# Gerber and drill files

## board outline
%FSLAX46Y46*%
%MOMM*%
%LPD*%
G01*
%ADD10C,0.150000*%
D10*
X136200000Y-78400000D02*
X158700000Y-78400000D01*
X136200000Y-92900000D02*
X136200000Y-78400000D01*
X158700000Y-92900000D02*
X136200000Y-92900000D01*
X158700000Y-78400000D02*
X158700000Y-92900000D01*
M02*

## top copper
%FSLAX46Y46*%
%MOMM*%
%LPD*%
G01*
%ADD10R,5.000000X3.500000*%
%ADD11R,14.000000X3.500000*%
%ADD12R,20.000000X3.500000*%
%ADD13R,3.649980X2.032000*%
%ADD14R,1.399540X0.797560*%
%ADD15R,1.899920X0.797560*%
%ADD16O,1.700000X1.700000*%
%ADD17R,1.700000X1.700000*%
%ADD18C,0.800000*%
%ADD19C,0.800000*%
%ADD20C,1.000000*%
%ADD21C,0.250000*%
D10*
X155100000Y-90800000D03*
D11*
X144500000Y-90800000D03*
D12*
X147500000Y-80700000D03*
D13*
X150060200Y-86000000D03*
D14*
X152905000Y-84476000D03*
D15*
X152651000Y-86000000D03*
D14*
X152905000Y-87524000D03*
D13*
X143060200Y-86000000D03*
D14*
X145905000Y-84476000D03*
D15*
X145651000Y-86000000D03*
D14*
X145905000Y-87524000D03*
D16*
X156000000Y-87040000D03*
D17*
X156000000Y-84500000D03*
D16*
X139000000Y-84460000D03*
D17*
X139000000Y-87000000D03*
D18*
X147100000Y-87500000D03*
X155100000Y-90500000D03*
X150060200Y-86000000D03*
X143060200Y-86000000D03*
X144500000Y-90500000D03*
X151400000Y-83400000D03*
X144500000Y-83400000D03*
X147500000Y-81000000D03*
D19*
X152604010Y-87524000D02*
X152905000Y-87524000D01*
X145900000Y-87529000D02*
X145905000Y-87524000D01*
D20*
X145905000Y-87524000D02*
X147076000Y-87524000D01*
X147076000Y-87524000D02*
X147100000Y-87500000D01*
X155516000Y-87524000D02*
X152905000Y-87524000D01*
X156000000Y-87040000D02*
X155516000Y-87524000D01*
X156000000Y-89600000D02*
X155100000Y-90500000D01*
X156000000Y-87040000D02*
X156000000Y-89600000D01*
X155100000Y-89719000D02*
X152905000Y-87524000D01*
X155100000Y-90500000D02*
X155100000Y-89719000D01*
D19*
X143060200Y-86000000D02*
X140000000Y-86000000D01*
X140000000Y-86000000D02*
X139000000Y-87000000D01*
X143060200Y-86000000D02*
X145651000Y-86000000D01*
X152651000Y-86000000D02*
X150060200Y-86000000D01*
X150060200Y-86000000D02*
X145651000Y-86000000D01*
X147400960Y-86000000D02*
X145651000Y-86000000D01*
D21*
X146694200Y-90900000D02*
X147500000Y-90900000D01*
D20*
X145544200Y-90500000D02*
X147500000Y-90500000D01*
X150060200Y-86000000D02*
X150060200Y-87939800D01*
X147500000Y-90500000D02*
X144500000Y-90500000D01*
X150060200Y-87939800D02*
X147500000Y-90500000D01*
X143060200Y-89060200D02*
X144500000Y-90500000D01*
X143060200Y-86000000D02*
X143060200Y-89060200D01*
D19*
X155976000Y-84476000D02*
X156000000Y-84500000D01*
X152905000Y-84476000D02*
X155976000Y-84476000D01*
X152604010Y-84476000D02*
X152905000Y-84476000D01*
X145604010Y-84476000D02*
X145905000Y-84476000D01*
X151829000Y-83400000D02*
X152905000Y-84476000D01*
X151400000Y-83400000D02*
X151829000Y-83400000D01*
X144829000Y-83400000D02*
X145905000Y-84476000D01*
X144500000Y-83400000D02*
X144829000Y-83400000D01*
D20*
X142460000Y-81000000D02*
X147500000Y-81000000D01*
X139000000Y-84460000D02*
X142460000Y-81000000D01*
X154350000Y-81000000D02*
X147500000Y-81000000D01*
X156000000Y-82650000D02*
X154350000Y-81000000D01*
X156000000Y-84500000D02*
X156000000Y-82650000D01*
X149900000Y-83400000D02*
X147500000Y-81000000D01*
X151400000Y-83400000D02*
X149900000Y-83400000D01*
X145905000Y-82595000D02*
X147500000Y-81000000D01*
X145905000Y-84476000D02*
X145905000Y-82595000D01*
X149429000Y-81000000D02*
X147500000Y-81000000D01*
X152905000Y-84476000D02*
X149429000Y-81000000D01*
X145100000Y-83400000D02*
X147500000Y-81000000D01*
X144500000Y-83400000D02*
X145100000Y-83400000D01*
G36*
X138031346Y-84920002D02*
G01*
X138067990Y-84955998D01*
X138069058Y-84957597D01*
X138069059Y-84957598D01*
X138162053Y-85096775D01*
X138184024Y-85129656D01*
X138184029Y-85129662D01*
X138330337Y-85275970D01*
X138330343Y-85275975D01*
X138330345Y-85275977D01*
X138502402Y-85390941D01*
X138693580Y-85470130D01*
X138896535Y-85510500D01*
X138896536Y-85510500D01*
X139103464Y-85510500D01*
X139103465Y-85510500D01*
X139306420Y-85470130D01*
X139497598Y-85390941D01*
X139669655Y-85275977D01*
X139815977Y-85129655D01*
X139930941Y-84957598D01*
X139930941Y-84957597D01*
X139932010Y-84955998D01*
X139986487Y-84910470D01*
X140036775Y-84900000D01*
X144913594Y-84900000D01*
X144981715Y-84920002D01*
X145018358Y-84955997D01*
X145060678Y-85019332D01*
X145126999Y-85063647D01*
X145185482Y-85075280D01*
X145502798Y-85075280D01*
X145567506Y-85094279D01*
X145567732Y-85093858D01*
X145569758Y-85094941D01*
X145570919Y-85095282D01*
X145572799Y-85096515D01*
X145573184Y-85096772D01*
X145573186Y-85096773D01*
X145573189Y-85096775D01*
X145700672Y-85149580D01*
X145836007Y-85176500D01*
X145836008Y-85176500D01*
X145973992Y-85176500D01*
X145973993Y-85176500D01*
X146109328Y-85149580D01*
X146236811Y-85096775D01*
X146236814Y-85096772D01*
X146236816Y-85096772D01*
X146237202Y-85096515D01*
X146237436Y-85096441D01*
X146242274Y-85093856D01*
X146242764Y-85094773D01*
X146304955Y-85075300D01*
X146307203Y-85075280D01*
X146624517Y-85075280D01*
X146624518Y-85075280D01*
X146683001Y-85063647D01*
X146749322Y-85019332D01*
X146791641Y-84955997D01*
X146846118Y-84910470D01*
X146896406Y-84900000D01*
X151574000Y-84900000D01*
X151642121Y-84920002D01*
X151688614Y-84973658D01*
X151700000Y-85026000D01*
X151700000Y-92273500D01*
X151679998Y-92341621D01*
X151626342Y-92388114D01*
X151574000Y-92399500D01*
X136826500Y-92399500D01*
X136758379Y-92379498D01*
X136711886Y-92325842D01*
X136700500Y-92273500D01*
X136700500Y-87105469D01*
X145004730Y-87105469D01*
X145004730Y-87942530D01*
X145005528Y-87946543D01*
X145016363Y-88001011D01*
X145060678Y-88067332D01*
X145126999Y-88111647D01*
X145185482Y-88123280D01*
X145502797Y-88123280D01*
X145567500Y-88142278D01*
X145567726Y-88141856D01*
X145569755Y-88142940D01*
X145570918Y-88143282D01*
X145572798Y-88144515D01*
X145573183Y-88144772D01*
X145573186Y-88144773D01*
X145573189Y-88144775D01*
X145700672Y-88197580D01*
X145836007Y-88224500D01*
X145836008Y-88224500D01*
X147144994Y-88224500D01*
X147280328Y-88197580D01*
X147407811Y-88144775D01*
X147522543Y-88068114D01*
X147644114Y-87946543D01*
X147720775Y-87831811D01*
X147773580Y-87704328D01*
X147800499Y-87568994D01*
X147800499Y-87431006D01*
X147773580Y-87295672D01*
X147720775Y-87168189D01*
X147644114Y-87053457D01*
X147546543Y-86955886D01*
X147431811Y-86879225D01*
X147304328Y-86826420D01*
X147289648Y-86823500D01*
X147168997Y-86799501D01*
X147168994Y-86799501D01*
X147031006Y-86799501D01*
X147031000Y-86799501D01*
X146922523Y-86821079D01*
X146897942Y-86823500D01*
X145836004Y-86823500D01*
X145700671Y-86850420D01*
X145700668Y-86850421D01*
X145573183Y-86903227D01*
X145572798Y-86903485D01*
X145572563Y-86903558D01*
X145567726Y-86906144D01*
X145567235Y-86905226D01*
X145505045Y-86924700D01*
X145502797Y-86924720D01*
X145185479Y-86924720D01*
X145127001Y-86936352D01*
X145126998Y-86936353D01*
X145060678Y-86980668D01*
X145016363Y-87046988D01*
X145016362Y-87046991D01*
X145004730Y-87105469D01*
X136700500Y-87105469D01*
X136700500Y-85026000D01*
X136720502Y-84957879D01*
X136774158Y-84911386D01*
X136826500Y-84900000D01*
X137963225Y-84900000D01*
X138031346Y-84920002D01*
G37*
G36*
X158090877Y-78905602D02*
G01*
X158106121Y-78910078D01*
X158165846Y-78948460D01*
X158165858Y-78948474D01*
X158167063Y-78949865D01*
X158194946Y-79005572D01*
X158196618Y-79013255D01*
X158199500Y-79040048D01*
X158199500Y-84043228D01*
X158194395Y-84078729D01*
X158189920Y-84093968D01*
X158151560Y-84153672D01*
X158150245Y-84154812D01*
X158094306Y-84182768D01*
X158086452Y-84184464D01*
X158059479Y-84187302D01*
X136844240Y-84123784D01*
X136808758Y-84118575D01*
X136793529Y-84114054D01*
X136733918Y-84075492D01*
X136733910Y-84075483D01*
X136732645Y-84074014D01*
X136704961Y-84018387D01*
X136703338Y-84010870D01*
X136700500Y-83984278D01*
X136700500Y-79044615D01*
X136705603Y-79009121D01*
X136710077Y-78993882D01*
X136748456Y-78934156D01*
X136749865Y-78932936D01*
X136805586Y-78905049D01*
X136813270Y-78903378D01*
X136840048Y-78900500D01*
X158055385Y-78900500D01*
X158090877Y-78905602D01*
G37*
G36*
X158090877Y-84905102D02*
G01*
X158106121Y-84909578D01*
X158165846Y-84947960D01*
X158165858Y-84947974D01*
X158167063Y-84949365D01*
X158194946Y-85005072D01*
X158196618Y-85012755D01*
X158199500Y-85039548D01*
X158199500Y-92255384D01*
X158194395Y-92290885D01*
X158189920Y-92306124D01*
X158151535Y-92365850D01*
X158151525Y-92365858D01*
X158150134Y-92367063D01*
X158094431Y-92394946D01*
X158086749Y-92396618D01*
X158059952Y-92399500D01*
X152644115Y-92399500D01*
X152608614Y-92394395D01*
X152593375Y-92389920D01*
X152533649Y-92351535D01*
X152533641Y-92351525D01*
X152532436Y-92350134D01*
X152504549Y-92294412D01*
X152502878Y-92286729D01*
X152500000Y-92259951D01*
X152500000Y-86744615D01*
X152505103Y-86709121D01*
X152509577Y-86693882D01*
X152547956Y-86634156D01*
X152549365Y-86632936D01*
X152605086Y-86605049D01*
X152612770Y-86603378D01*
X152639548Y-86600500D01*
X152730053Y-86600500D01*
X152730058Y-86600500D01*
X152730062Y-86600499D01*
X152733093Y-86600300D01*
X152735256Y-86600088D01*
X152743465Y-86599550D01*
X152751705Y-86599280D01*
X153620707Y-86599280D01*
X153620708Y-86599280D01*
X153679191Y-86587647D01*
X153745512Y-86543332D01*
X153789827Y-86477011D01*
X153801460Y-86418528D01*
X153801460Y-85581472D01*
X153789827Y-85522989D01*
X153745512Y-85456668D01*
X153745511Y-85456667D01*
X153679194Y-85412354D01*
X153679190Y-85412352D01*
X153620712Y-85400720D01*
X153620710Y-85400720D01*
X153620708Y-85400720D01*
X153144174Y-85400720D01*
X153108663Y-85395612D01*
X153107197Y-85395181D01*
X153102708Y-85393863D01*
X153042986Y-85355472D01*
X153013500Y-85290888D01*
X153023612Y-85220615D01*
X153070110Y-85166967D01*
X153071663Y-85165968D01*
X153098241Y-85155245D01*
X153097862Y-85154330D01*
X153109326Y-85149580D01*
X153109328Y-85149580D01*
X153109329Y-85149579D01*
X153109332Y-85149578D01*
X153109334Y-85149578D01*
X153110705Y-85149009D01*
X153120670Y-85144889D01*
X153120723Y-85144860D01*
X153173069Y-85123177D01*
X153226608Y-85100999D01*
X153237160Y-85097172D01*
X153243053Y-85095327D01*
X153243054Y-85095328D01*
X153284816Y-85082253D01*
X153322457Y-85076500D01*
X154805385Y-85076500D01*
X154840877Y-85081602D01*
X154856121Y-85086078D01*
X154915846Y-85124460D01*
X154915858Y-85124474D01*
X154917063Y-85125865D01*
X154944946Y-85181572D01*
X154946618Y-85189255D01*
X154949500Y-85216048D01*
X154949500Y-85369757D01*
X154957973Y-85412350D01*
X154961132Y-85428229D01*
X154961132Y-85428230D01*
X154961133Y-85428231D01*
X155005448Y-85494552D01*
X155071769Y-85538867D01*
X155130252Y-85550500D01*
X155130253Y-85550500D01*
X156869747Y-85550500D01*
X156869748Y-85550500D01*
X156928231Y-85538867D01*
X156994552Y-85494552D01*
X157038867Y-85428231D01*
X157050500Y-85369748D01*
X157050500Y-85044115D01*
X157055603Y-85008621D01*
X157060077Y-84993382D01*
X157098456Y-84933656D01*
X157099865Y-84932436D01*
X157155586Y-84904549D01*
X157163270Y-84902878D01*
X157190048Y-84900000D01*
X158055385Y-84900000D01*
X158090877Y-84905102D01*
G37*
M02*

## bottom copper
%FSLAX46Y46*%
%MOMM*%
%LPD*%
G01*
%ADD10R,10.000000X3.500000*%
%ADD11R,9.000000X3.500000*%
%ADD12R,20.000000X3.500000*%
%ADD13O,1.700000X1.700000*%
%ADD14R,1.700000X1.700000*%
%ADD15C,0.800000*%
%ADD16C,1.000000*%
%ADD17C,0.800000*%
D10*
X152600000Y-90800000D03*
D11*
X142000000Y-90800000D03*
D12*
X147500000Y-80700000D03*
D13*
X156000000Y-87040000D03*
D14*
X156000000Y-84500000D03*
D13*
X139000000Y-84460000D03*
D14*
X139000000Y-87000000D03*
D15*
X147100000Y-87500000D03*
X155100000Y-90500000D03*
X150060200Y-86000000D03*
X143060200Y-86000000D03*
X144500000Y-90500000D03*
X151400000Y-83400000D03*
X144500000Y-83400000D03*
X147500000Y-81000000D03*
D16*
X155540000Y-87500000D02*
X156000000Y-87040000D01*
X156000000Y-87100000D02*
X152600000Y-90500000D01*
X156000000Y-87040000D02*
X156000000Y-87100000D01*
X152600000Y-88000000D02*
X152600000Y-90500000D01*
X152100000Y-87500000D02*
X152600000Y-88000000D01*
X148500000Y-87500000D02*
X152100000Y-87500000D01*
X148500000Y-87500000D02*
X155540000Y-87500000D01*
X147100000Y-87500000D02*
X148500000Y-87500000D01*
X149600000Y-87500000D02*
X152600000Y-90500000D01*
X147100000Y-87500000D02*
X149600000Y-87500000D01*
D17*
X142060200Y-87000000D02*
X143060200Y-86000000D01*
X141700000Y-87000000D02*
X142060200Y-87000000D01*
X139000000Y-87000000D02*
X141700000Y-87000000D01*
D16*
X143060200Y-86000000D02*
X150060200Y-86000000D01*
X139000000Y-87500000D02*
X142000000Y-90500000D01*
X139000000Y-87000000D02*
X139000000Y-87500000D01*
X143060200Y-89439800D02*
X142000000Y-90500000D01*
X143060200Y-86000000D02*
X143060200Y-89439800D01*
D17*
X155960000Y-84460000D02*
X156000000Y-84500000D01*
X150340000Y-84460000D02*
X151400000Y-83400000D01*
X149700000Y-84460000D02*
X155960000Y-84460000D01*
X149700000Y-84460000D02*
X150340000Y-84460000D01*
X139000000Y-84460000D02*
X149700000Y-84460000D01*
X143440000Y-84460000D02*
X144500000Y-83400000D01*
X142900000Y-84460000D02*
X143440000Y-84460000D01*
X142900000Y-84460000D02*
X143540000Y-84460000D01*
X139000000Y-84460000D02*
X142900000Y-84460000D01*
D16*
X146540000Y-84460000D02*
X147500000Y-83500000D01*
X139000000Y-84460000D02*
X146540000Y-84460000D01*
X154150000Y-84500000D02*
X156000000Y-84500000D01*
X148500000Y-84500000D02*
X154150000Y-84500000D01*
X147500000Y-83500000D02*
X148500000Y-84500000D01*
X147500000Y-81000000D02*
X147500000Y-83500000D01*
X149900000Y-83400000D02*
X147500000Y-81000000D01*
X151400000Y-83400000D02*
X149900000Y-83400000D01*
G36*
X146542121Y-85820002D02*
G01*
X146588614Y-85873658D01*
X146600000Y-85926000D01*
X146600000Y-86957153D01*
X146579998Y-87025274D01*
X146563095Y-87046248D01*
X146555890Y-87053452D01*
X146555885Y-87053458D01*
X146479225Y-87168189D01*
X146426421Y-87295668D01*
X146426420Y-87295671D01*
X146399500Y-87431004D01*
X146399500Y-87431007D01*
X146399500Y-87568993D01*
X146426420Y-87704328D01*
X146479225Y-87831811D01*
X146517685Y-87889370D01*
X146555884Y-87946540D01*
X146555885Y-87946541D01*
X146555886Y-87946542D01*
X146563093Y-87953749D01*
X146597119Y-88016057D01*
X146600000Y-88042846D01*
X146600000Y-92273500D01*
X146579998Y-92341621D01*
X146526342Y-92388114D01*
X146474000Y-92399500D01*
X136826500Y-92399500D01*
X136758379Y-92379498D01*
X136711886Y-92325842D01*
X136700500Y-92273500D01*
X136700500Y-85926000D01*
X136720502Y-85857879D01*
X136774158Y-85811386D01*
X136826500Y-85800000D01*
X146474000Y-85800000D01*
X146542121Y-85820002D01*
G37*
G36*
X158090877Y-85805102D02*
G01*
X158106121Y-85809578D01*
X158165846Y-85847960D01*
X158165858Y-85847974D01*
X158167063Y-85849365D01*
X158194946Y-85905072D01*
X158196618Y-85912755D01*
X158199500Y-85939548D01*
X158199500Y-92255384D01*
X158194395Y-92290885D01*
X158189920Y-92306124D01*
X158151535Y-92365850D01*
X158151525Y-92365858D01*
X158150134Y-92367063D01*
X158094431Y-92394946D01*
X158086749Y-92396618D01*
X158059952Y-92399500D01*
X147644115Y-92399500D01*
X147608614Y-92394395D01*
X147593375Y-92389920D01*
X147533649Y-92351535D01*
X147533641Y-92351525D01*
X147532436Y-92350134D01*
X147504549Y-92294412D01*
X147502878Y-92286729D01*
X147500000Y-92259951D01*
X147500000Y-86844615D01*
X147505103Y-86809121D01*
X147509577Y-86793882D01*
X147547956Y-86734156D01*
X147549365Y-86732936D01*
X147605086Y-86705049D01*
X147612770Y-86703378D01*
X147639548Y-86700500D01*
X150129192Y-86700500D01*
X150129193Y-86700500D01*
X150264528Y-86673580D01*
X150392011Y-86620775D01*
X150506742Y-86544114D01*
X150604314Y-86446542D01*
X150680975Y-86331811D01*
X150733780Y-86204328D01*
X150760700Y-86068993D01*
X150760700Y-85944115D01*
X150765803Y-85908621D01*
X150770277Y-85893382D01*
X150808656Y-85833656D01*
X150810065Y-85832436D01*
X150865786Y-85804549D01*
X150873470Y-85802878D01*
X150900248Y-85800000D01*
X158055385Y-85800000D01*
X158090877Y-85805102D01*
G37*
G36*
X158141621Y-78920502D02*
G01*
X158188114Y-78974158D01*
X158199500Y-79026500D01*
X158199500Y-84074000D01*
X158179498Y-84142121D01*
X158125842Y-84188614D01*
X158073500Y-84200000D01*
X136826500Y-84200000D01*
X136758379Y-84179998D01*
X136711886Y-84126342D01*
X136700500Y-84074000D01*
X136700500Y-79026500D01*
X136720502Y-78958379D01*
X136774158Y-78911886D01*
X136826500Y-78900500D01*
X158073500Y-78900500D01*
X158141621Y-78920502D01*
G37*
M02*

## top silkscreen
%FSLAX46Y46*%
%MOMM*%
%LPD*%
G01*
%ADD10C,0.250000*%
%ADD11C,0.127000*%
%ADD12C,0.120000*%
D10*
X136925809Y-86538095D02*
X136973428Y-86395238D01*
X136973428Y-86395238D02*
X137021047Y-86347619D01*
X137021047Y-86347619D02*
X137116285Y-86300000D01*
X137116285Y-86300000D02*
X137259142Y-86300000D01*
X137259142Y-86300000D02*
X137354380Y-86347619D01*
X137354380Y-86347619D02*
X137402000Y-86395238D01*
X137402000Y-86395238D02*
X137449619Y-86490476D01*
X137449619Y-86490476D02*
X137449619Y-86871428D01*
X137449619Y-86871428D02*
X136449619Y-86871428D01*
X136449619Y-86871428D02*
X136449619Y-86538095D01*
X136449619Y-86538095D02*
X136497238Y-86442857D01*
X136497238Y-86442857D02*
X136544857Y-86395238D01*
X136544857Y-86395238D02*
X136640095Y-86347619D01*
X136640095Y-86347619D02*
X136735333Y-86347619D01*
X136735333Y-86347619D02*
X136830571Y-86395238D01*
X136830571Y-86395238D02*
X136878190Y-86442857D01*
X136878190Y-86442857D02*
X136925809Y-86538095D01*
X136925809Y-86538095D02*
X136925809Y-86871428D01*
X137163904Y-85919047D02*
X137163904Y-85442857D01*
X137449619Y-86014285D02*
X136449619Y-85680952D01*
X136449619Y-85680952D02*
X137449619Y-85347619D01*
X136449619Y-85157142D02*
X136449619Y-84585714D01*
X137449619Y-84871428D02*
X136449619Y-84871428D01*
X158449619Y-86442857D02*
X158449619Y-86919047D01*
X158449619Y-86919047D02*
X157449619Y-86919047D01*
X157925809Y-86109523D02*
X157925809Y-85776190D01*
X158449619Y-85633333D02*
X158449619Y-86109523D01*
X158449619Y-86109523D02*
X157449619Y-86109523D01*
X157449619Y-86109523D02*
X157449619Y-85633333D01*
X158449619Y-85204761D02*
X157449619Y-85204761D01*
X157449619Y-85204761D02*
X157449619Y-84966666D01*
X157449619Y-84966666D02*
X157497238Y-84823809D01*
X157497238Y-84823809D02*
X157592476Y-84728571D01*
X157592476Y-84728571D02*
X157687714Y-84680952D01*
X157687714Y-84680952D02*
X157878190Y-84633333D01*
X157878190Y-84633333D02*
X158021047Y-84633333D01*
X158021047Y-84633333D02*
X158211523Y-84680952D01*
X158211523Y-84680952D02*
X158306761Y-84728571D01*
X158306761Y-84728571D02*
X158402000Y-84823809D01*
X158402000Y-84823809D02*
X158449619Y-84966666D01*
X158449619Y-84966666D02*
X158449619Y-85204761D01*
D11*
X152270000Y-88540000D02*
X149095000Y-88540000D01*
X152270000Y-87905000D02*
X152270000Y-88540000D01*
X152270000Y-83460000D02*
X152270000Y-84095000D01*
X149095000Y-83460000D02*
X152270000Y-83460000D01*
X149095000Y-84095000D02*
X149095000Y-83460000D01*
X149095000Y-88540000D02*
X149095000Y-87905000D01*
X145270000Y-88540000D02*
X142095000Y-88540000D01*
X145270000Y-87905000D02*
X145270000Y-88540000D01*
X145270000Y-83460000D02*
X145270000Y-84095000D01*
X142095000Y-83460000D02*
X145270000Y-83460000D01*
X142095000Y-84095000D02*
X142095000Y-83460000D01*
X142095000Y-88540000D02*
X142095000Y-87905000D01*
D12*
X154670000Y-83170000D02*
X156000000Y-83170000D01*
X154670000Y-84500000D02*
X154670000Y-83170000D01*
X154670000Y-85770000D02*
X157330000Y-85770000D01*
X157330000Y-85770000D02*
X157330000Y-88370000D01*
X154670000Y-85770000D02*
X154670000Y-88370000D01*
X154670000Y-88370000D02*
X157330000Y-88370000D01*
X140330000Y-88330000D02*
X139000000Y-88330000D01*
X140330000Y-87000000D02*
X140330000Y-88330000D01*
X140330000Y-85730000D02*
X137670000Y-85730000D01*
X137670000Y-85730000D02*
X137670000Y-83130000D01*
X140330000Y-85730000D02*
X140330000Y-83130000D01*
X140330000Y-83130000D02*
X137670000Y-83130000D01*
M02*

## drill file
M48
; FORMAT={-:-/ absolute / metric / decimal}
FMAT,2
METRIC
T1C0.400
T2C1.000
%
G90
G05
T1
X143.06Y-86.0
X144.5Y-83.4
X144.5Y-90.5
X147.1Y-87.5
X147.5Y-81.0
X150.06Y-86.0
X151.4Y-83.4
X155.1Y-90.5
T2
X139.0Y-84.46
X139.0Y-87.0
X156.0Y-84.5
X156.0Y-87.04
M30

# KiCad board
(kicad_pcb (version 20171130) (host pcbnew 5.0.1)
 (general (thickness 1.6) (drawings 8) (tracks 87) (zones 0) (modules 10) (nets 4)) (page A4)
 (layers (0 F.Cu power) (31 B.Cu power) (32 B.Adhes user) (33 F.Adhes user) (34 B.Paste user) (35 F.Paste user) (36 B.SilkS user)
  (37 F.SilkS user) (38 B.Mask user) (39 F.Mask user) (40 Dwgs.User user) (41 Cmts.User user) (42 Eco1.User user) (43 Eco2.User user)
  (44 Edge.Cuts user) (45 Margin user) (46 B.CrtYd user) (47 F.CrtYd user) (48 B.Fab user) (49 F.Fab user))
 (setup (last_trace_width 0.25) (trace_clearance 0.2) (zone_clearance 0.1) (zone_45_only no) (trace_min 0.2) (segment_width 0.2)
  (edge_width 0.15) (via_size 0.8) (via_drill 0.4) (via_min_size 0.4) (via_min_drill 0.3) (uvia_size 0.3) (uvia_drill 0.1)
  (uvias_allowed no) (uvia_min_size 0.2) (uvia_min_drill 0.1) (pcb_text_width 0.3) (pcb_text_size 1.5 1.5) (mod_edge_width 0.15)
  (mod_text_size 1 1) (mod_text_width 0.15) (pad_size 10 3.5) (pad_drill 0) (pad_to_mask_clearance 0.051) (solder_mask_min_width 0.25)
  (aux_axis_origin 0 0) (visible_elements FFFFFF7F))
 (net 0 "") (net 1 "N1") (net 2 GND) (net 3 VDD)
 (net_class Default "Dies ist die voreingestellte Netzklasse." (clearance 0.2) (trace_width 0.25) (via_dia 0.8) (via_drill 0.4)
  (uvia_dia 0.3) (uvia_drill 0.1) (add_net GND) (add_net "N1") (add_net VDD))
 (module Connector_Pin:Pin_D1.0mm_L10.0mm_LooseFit (layer F.Cu) (at 155.1 90.8)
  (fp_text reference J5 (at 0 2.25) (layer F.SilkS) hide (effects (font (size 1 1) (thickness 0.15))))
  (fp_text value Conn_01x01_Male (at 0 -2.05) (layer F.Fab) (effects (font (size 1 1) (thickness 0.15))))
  (pad 1 smd rect (at 0 0) (size 5 3.5) (layers F.Cu F.Paste F.Mask) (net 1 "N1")))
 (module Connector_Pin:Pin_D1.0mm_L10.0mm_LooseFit (layer F.Cu) (at 144.5 90.8)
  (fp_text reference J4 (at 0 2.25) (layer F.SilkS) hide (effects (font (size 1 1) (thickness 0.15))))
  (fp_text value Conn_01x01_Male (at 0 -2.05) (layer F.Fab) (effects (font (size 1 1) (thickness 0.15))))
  (pad 1 smd rect (at 0 0) (size 14 3.5) (layers F.Cu F.Paste F.Mask) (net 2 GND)))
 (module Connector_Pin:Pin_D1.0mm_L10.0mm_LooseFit (layer B.Cu) (at 152.6 90.8)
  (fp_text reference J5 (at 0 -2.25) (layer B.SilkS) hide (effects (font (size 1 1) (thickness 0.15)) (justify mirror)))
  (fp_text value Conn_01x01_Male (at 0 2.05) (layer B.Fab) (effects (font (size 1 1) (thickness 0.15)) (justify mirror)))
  (pad 1 smd rect (at 0 0) (size 10 3.5) (layers B.Cu B.Paste B.Mask) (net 1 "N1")))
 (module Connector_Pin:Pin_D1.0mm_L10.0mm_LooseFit (layer B.Cu) (at 142 90.8)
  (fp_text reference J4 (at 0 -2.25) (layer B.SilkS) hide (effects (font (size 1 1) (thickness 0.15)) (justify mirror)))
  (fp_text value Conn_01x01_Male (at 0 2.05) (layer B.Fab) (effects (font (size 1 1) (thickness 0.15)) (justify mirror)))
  (pad 1 smd rect (at 0 0) (size 9 3.5) (layers B.Cu B.Paste B.Mask) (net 2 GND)))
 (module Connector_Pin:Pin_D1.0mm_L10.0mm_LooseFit (layer B.Cu) (at 147.5 80.7)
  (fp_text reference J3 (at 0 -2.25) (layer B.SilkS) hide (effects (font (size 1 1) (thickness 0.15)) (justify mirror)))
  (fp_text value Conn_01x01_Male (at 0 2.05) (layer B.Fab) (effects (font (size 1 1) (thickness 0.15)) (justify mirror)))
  (pad 1 smd rect (at 0 0) (size 20 3.5) (layers B.Cu B.Paste B.Mask) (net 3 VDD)))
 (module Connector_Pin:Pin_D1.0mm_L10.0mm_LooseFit (layer F.Cu) (at 147.5 80.7)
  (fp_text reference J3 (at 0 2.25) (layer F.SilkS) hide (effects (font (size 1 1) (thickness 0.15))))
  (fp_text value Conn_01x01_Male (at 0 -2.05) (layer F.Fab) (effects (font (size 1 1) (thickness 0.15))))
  (pad 1 smd rect (at 0 0) (size 20 3.5) (layers F.Cu F.Paste F.Mask) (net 3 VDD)))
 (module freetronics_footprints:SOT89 (layer F.Cu) (at 151 86 90)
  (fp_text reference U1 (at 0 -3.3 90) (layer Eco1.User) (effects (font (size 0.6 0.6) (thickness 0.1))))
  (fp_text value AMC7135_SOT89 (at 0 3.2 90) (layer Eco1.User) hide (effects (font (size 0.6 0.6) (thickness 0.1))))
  (fp_line (start -2.54 1.27) (end -2.54 -1.905) (layer F.SilkS) (width 0.127))
  (fp_line (start -1.905 1.27) (end -2.54 1.27) (layer F.SilkS) (width 0.127))
  (fp_line (start 2.54 1.27) (end 1.905 1.27) (layer F.SilkS) (width 0.127))
  (fp_line (start 2.54 -1.905) (end 2.54 1.27) (layer F.SilkS) (width 0.127))
  (fp_line (start 1.905 -1.905) (end 2.54 -1.905) (layer F.SilkS) (width 0.127))
  (fp_line (start -2.54 -1.905) (end -1.905 -1.905) (layer F.SilkS) (width 0.127))
  (pad 2 smd rect (at 0 -0.9398 90) (size 2.032 3.64998) (layers F.Cu F.Paste F.Mask) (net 2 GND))
  (pad 3 smd rect (at 1.524 1.905 90) (size 0.79756 1.39954) (layers F.Cu F.Paste F.Mask) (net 3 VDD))
  (pad 2 smd rect (at 0 1.651 90) (size 0.79756 1.89992) (layers F.Cu F.Paste F.Mask) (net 2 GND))
  (pad 1 smd rect (at -1.524 1.905 90) (size 0.79756 1.39954) (layers F.Cu F.Paste F.Mask) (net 1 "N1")))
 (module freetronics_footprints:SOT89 (layer F.Cu) (at 144 86 90)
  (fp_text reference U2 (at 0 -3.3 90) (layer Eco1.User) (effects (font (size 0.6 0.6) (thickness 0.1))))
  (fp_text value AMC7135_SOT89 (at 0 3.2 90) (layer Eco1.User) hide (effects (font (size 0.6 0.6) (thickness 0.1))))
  (fp_line (start -2.54 1.27) (end -2.54 -1.905) (layer F.SilkS) (width 0.127))
  (fp_line (start -1.905 1.27) (end -2.54 1.27) (layer F.SilkS) (width 0.127))
  (fp_line (start 2.54 1.27) (end 1.905 1.27) (layer F.SilkS) (width 0.127))
  (fp_line (start 2.54 -1.905) (end 2.54 1.27) (layer F.SilkS) (width 0.127))
  (fp_line (start 1.905 -1.905) (end 2.54 -1.905) (layer F.SilkS) (width 0.127))
  (fp_line (start -2.54 -1.905) (end -1.905 -1.905) (layer F.SilkS) (width 0.127))
  (pad 2 smd rect (at 0 -0.9398 90) (size 2.032 3.64998) (layers F.Cu F.Paste F.Mask) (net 2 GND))
  (pad 3 smd rect (at 1.524 1.905 90) (size 0.79756 1.39954) (layers F.Cu F.Paste F.Mask) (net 3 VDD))
  (pad 2 smd rect (at 0 1.651 90) (size 0.79756 1.89992) (layers F.Cu F.Paste F.Mask) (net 2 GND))
  (pad 1 smd rect (at -1.524 1.905 90) (size 0.79756 1.39954) (layers F.Cu F.Paste F.Mask) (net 1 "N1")))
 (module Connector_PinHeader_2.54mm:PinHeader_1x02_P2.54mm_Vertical (layer F.Cu) (at 156 84.5)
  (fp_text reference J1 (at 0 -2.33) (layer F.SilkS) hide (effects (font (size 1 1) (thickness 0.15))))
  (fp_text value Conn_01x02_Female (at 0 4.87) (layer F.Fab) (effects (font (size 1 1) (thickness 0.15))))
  (fp_line (start -1.33 -1.33) (end 0 -1.33) (layer F.SilkS) (width 0.12))
  (fp_line (start -1.33 0) (end -1.33 -1.33) (layer F.SilkS) (width 0.12))
  (fp_line (start -1.33 1.27) (end 1.33 1.27) (layer F.SilkS) (width 0.12))
  (fp_line (start 1.33 1.27) (end 1.33 3.87) (layer F.SilkS) (width 0.12))
  (fp_line (start -1.33 1.27) (end -1.33 3.87) (layer F.SilkS) (width 0.12))
  (fp_line (start -1.33 3.87) (end 1.33 3.87) (layer F.SilkS) (width 0.12))
  (pad 2 thru_hole oval (at 0 2.54) (size 1.7 1.7) (drill 1) (layers *.Cu *.Mask) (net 1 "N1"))
  (pad 1 thru_hole rect (at 0 0) (size 1.7 1.7) (drill 1) (layers *.Cu *.Mask) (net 3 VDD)))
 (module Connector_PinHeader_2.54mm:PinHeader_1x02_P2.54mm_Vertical (layer F.Cu) (at 139 87 180)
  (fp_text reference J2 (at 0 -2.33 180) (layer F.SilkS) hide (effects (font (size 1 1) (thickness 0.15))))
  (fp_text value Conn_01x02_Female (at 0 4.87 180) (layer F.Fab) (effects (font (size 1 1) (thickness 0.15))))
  (fp_line (start -1.33 -1.33) (end 0 -1.33) (layer F.SilkS) (width 0.12))
  (fp_line (start -1.33 0) (end -1.33 -1.33) (layer F.SilkS) (width 0.12))
  (fp_line (start -1.33 1.27) (end 1.33 1.27) (layer F.SilkS) (width 0.12))
  (fp_line (start 1.33 1.27) (end 1.33 3.87) (layer F.SilkS) (width 0.12))
  (fp_line (start -1.33 1.27) (end -1.33 3.87) (layer F.SilkS) (width 0.12))
  (fp_line (start -1.33 3.87) (end 1.33 3.87) (layer F.SilkS) (width 0.12))
  (pad 2 thru_hole oval (at 0 2.54 180) (size 1.7 1.7) (drill 1) (layers *.Cu *.Mask) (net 3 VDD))
  (pad 1 thru_hole rect (at 0 0 180) (size 1.7 1.7) (drill 1) (layers *.Cu *.Mask) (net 2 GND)))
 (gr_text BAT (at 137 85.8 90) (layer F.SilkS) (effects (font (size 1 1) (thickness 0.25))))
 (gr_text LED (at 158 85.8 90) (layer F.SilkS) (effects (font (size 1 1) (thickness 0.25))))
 (gr_line (start 136.2 78.4) (end 158.7 78.4) (layer Edge.Cuts) (width 0.15))
 (gr_line (start 136.2 92.9) (end 136.2 78.4) (layer Edge.Cuts) (width 0.15))
 (gr_line (start 158.7 92.9) (end 136.2 92.9) (layer Edge.Cuts) (width 0.15))
 (gr_line (start 158.7 78.4) (end 158.7 92.9) (layer Edge.Cuts) (width 0.15))
 (segment (start 152.60401 87.524) (end 152.905 87.524) (width 0.8) (layer F.Cu) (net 1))
 (segment (start 145.9 87.529) (end 145.905 87.524) (width 0.8) (layer F.Cu) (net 1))
 (via (at 147.1 87.5) (size 0.8) (drill 0.4) (layers F.Cu B.Cu) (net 1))
 (segment (start 145.905 87.524) (end 147.076 87.524) (width 1) (layer F.Cu) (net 1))
 (segment (start 147.076 87.524) (end 147.1 87.5) (width 1) (layer F.Cu) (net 1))
 (segment (start 155.54 87.5) (end 156 87.04) (width 1) (layer B.Cu) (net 1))
 (segment (start 155.516 87.524) (end 152.905 87.524) (width 1) (layer F.Cu) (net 1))
 (segment (start 156 87.04) (end 155.516 87.524) (width 1) (layer F.Cu) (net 1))
 (segment (start 156 87.1) (end 152.6 90.5) (width 1) (layer B.Cu) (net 1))
 (segment (start 156 87.04) (end 156 87.1) (width 1) (layer B.Cu) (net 1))
 (segment (start 152.6 88) (end 152.6 90.5) (width 1) (layer B.Cu) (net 1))
 (segment (start 152.1 87.5) (end 152.6 88) (width 1) (layer B.Cu) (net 1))
 (segment (start 148.5 87.5) (end 152.1 87.5) (width 1) (layer B.Cu) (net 1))
 (segment (start 148.5 87.5) (end 155.54 87.5) (width 1) (layer B.Cu) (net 1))
 (segment (start 147.1 87.5) (end 148.5 87.5) (width 1) (layer B.Cu) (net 1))
 (segment (start 149.6 87.5) (end 152.6 90.5) (width 1) (layer B.Cu) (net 1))
 (segment (start 147.1 87.5) (end 149.6 87.5) (width 1) (layer B.Cu) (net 1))
 (segment (start 156 89.6) (end 155.1 90.5) (width 1) (layer F.Cu) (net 1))
 (segment (start 156 87.04) (end 156 89.6) (width 1) (layer F.Cu) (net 1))
 (via (at 155.1 90.5) (size 0.8) (drill 0.4) (layers F.Cu B.Cu) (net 1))
 (segment (start 155.1 89.719) (end 152.905 87.524) (width 1) (layer F.Cu) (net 1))
 (segment (start 155.1 90.5) (end 155.1 89.719) (width 1) (layer F.Cu) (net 1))
 (segment (start 143.0602 86) (end 140 86) (width 0.8) (layer F.Cu) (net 2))
 (segment (start 140 86) (end 139 87) (width 0.8) (layer F.Cu) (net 2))
 (segment (start 143.0602 86) (end 145.651 86) (width 0.8) (layer F.Cu) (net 2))
 (segment (start 152.651 86) (end 150.0602 86) (width 0.8) (layer F.Cu) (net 2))
 (segment (start 150.0602 86) (end 145.651 86) (width 0.8) (layer F.Cu) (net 2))
 (segment (start 147.40096 86) (end 145.651 86) (width 0.8) (layer F.Cu) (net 2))
 (via (at 150.0602 86) (size 0.8) (drill 0.4) (layers F.Cu B.Cu) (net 2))
 (segment (start 142.0602 87) (end 143.0602 86) (width 0.8) (layer B.Cu) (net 2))
 (segment (start 141.7 87) (end 142.0602 87) (width 0.8) (layer B.Cu) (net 2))
 (via (at 143.0602 86) (size 0.8) (drill 0.4) (layers F.Cu B.Cu) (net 2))
 (segment (start 139 87) (end 141.7 87) (width 0.8) (layer B.Cu) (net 2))
 (segment (start 146.6942 90.9) (end 147.5 90.9) (width 0.25) (layer F.Cu) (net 2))
 (segment (start 143.0602 86) (end 150.0602 86) (width 1) (layer B.Cu) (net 2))
 (segment (start 145.5442 90.5) (end 147.5 90.5) (width 1) (layer F.Cu) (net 2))
 (segment (start 150.0602 86) (end 150.0602 87.9398) (width 1) (layer F.Cu) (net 2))
 (via (at 144.5 90.5) (size 0.8) (drill 0.4) (layers F.Cu B.Cu) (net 2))
 (segment (start 147.5 90.5) (end 144.5 90.5) (width 1) (layer F.Cu) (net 2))
 (segment (start 150.0602 87.9398) (end 147.5 90.5) (width 1) (layer F.Cu) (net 2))
 (segment (start 143.0602 89.0602) (end 144.5 90.5) (width 1) (layer F.Cu) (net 2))
 (segment (start 143.0602 86) (end 143.0602 89.0602) (width 1) (layer F.Cu) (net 2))
 (segment (start 139 87.5) (end 142 90.5) (width 1) (layer B.Cu) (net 2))
 (segment (start 139 87) (end 139 87.5) (width 1) (layer B.Cu) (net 2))
 (segment (start 143.0602 89.4398) (end 142 90.5) (width 1) (layer B.Cu) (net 2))
 (segment (start 143.0602 86) (end 143.0602 89.4398) (width 1) (layer B.Cu) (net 2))
 (segment (start 155.976 84.476) (end 156 84.5) (width 0.8) (layer F.Cu) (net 3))
 (segment (start 152.905 84.476) (end 155.976 84.476) (width 0.8) (layer F.Cu) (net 3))
 (segment (start 152.60401 84.476) (end 152.905 84.476) (width 0.8) (layer F.Cu) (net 3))
 (segment (start 155.96 84.46) (end 156 84.5) (width 0.8) (layer B.Cu) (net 3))
 (segment (start 145.60401 84.476) (end 145.905 84.476) (width 0.8) (layer F.Cu) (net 3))
 (segment (start 150.34 84.46) (end 151.4 83.4) (width 0.8) (layer B.Cu) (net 3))
 (segment (start 149.7 84.46) (end 155.96 84.46) (width 0.8) (layer B.Cu) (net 3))
 (via (at 151.4 83.4) (size 0.8) (drill 0.4) (layers F.Cu B.Cu) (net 3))
 (segment (start 149.7 84.46) (end 150.34 84.46) (width 0.8) (layer B.Cu) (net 3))
 (segment (start 139 84.46) (end 149.7 84.46) (width 0.8) (layer B.Cu) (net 3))
 (segment (start 151.829 83.4) (end 152.905 84.476) (width 0.8) (layer F.Cu) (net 3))
 (segment (start 151.4 83.4) (end 151.829 83.4) (width 0.8) (layer F.Cu) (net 3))
 (via (at 144.5 83.4) (size 0.8) (drill 0.4) (layers F.Cu B.Cu) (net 3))
 (segment (start 143.44 84.46) (end 144.5 83.4) (width 0.8) (layer B.Cu) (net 3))
 (segment (start 142.9 84.46) (end 143.44 84.46) (width 0.8) (layer B.Cu) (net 3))
 (segment (start 142.9 84.46) (end 143.54 84.46) (width 0.8) (layer B.Cu) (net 3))
 (segment (start 139 84.46) (end 142.9 84.46) (width 0.8) (layer B.Cu) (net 3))
 (segment (start 144.829 83.4) (end 145.905 84.476) (width 0.8) (layer F.Cu) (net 3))
 (segment (start 144.5 83.4) (end 144.829 83.4) (width 0.8) (layer F.Cu) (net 3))
 (segment (start 142.46 81) (end 147.5 81) (width 1) (layer F.Cu) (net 3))
 (segment (start 139 84.46) (end 142.46 81) (width 1) (layer F.Cu) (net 3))
 (segment (start 154.35 81) (end 147.5 81) (width 1) (layer F.Cu) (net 3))
 (segment (start 156 82.65) (end 154.35 81) (width 1) (layer F.Cu) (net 3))
 (segment (start 156 84.5) (end 156 82.65) (width 1) (layer F.Cu) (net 3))
 (segment (start 149.9 83.4) (end 147.5 81) (width 1) (layer F.Cu) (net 3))
 (segment (start 151.4 83.4) (end 149.9 83.4) (width 1) (layer F.Cu) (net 3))
 (segment (start 145.905 82.595) (end 147.5 81) (width 1) (layer F.Cu) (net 3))
 (segment (start 145.905 84.476) (end 145.905 82.595) (width 1) (layer F.Cu) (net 3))
 (segment (start 149.429 81) (end 147.5 81) (width 1) (layer F.Cu) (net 3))
 (segment (start 152.905 84.476) (end 149.429 81) (width 1) (layer F.Cu) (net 3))
 (segment (start 146.54 84.46) (end 147.5 83.5) (width 1) (layer B.Cu) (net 3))
 (segment (start 139 84.46) (end 146.54 84.46) (width 1) (layer B.Cu) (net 3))
 (segment (start 154.15 84.5) (end 156 84.5) (width 1) (layer B.Cu) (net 3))
 (segment (start 148.5 84.5) (end 154.15 84.5) (width 1) (layer B.Cu) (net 3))
 (segment (start 147.5 83.5) (end 148.5 84.5) (width 1) (layer B.Cu) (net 3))
 (segment (start 147.5 81) (end 147.5 83.5) (width 1) (layer B.Cu) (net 3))
 (segment (start 149.9 83.4) (end 147.5 81) (width 1) (layer B.Cu) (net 3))
 (segment (start 151.4 83.4) (end 149.9 83.4) (width 1) (layer B.Cu) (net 3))
 (via (at 147.5 81) (size 0.8) (drill 0.4) (layers F.Cu B.Cu) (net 3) (status 1000000))
 (segment (start 145.1 83.4) (end 147.5 81) (width 1) (layer F.Cu) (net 3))
 (segment (start 144.5 83.4) (end 145.1 83.4) (width 1) (layer F.Cu) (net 3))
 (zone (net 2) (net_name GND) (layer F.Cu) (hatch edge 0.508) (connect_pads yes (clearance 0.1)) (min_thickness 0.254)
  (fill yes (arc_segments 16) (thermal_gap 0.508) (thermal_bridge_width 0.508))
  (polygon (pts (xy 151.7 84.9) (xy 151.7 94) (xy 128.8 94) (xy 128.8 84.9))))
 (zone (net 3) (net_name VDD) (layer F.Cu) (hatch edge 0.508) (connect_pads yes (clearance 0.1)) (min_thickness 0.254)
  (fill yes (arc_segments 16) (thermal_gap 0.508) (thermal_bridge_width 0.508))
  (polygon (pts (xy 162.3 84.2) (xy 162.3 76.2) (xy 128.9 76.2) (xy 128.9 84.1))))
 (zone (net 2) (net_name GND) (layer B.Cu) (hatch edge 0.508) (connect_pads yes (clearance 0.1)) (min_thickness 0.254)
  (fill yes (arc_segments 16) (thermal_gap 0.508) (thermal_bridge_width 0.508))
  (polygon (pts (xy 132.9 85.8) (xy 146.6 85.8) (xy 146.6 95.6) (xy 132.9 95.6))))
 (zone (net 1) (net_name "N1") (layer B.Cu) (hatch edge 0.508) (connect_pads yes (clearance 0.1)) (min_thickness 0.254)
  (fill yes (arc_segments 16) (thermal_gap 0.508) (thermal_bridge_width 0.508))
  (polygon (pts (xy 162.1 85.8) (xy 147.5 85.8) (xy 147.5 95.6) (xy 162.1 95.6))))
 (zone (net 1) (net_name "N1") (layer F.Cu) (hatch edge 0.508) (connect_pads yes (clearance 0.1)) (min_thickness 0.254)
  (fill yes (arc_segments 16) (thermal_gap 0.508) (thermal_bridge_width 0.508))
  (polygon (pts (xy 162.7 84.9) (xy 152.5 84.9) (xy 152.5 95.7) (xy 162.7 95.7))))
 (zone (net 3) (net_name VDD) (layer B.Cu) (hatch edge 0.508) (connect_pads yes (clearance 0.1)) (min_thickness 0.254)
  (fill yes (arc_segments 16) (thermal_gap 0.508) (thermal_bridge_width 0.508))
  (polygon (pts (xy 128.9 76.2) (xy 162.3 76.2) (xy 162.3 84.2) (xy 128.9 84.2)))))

